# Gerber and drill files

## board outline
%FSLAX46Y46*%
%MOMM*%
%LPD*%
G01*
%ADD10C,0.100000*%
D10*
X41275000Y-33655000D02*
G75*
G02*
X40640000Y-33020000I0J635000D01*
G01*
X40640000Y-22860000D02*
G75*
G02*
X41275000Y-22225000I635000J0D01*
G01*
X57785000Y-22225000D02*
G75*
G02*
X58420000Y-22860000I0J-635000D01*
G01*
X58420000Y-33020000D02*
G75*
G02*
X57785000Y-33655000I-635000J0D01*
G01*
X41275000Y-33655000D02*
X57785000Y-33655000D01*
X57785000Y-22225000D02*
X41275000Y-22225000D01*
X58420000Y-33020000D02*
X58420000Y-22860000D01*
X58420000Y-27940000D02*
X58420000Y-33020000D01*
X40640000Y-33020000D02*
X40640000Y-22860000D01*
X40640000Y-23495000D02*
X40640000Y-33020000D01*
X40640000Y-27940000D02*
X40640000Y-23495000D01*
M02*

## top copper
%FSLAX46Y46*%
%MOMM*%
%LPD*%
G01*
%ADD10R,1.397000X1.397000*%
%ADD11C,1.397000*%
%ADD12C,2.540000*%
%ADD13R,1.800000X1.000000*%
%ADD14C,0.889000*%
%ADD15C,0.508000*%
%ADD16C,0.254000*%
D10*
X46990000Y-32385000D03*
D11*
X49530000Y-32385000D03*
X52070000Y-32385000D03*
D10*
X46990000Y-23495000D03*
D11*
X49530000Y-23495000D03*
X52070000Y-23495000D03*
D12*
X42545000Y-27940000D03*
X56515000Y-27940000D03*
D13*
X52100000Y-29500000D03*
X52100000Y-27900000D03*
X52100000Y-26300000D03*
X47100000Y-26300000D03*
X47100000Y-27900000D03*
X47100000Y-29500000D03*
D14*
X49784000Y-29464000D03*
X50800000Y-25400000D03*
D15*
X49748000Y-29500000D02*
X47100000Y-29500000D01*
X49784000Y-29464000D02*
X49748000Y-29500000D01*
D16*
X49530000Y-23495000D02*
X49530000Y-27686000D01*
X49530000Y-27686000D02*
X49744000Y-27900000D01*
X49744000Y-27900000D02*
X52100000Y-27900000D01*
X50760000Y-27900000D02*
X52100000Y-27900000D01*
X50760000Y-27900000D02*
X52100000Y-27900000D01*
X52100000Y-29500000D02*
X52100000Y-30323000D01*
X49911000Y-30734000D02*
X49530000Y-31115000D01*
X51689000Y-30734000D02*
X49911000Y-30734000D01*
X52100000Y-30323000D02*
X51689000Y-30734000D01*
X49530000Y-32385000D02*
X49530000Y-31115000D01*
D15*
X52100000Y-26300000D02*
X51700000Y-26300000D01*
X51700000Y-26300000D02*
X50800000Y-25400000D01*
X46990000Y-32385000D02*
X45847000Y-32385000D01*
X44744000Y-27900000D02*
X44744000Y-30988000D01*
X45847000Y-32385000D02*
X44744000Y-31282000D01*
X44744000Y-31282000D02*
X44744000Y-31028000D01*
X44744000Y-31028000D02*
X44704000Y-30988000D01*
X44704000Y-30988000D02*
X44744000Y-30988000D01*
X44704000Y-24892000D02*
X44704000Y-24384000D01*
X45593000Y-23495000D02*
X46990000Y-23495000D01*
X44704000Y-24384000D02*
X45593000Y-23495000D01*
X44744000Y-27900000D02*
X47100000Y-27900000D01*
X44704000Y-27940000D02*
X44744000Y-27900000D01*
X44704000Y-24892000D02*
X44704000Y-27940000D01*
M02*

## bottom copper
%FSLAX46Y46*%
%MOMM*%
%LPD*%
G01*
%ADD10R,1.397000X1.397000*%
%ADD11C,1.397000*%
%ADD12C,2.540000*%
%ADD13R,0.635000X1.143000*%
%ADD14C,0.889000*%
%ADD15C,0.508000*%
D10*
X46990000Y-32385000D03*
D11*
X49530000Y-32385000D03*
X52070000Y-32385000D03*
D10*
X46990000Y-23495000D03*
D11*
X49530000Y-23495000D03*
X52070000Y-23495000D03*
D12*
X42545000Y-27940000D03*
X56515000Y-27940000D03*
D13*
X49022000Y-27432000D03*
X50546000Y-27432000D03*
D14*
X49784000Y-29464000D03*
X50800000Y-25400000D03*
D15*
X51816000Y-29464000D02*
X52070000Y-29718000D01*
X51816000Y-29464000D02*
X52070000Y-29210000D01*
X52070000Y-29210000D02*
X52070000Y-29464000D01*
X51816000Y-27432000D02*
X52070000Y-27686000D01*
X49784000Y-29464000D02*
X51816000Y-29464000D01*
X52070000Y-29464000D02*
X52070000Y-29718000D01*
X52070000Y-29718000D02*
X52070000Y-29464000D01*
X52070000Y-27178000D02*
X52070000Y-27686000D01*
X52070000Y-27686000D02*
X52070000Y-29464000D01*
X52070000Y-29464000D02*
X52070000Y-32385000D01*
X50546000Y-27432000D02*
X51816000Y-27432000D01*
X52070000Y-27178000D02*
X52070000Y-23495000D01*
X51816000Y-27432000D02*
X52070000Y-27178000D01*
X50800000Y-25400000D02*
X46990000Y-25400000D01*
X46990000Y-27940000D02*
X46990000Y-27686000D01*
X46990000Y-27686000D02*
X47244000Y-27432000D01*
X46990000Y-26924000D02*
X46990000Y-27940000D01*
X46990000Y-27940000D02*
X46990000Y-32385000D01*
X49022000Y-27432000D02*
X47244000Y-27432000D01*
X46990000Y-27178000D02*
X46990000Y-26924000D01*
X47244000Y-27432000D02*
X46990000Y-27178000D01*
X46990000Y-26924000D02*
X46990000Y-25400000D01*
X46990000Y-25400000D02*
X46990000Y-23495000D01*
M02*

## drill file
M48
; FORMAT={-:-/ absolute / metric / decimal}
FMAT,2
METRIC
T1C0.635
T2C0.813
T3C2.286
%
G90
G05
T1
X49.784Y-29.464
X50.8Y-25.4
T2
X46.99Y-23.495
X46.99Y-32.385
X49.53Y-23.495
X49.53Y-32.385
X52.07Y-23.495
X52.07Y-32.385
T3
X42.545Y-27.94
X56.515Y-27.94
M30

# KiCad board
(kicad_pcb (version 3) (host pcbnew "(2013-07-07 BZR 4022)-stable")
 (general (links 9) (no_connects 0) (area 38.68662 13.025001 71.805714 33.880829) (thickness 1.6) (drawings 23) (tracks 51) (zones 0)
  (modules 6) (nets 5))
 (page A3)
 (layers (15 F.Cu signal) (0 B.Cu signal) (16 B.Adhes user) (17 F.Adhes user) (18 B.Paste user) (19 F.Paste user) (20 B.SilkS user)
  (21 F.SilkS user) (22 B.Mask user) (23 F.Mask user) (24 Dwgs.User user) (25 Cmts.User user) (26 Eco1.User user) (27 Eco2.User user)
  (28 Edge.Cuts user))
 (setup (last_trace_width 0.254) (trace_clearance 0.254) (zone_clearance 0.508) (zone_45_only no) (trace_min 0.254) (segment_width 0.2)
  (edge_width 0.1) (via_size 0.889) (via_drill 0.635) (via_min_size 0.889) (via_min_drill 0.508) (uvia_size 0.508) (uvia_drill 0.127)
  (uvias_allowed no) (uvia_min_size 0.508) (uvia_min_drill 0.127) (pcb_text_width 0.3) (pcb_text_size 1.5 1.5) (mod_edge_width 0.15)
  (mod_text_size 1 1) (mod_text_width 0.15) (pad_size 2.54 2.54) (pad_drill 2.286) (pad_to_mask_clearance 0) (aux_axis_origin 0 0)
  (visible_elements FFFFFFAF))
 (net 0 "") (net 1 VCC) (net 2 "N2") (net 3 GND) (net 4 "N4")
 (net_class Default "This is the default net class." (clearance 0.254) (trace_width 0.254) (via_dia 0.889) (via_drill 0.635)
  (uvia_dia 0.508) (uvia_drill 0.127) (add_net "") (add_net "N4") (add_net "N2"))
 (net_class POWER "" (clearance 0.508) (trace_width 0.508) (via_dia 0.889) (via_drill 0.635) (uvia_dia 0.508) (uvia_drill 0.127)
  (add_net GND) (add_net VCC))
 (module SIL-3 (layer F.Cu) (at 49.53 32.385)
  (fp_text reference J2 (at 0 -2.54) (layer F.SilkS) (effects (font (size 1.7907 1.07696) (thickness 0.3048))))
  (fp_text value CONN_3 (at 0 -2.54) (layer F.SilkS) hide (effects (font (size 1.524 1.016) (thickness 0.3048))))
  (pad 1 thru_hole rect (at -2.54 0) (size 1.397 1.397) (drill 0.8128) (layers *.Cu *.Mask F.SilkS) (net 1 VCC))
  (pad 2 thru_hole circle (at 0 0) (size 1.397 1.397) (drill 0.8128) (layers *.Cu *.Mask F.SilkS) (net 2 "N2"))
  (pad 3 thru_hole circle (at 2.54 0) (size 1.397 1.397) (drill 0.8128) (layers *.Cu *.Mask F.SilkS) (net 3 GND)))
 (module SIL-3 (layer F.Cu) (at 49.53 23.495)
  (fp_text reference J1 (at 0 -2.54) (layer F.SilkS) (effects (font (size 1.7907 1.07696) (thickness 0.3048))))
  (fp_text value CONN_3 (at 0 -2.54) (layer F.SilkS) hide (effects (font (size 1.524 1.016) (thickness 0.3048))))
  (pad 1 thru_hole rect (at -2.54 0) (size 1.397 1.397) (drill 0.8128) (layers *.Cu *.Mask F.SilkS) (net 1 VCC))
  (pad 2 thru_hole circle (at 0 0) (size 1.397 1.397) (drill 0.8128) (layers *.Cu *.Mask F.SilkS) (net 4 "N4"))
  (pad 3 thru_hole circle (at 2.54 0) (size 1.397 1.397) (drill 0.8128) (layers *.Cu *.Mask F.SilkS) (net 3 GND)))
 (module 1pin (layer F.Cu) (at 42.545 27.94)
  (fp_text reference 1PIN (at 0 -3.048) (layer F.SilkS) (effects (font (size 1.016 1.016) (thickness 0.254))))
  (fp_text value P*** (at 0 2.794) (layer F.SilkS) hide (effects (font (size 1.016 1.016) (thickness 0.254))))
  (pad 1 thru_hole circle (at 0 0) (size 2.54 2.54) (drill 2.286) (layers *.Cu *.Mask F.SilkS)))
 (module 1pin (layer F.Cu) (at 56.515 27.94)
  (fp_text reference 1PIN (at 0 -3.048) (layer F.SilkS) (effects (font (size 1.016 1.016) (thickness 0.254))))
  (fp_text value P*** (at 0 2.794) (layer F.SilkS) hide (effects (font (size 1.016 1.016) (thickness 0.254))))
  (pad 1 thru_hole circle (at 0 0) (size 2.54 2.54) (drill 2.286) (layers *.Cu *.Mask F.SilkS)))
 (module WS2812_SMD (layer F.Cu) (at 52.1 29.5)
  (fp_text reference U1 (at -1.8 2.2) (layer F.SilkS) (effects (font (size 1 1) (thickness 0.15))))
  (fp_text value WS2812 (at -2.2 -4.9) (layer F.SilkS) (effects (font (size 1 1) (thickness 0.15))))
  (pad 1 smd rect (at 0 0) (size 1.8 1) (layers F.Cu F.Paste F.Mask) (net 2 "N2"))
  (pad 2 smd rect (at 0 -1.6) (size 1.8 1) (layers F.Cu F.Paste F.Mask) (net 4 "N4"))
  (pad 3 smd rect (at 0 -3.2) (size 1.8 1) (layers F.Cu F.Paste F.Mask) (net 1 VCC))
  (pad 4 smd rect (at -5 -3.2) (size 1.8 1) (layers F.Cu F.Paste F.Mask))
  (pad 5 smd rect (at -5 -1.6) (size 1.8 1) (layers F.Cu F.Paste F.Mask) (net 1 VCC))
  (pad 6 smd rect (at -5 0) (size 1.8 1) (layers F.Cu F.Paste F.Mask) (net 3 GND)))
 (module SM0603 (layer B.Cu) (at 49.784 27.432)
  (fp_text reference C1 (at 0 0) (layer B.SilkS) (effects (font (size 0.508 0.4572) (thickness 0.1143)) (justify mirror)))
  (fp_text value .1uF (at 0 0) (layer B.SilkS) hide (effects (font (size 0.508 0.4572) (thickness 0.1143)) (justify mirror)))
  (pad 1 smd rect (at -0.762 0) (size 0.635 1.143) (layers B.Cu B.Paste B.Mask) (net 1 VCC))
  (pad 2 smd rect (at 0.762 0) (size 0.635 1.143) (layers B.Cu B.Paste B.Mask) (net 3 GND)))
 (gr_arc (start 41.275 33.02) (end 41.275 33.655) (angle 90) (layer Edge.Cuts) (width 0.1))
 (gr_arc (start 41.275 22.86) (end 40.64 22.86) (angle 90) (layer Edge.Cuts) (width 0.1))
 (gr_arc (start 57.785 22.86) (end 57.785 22.225) (angle 90) (layer Edge.Cuts) (width 0.1))
 (gr_arc (start 57.785 33.02) (end 58.42 33.02) (angle 90) (layer Edge.Cuts) (width 0.1))
 (gr_line (start 41.275 33.655) (end 57.785 33.655) (angle 90) (layer Edge.Cuts) (width 0.1))
 (gr_line (start 57.785 22.225) (end 41.275 22.225) (angle 90) (layer Edge.Cuts) (width 0.1))
 (gr_line (start 58.42 33.02) (end 58.42 22.86) (angle 90) (layer Edge.Cuts) (width 0.1))
 (gr_line (start 58.42 27.94) (end 58.42 33.02) (angle 90) (layer Edge.Cuts) (width 0.1))
 (gr_line (start 40.64 33.02) (end 40.64 22.86) (angle 90) (layer Edge.Cuts) (width 0.1))
 (gr_line (start 40.64 23.495) (end 40.64 33.02) (angle 90) (layer Edge.Cuts) (width 0.1))
 (gr_line (start 40.64 27.94) (end 40.64 23.495) (angle 90) (layer Edge.Cuts) (width 0.1))
 (segment (start 51.816 29.464) (end 52.07 29.718) (width 0.508) (layer B.Cu) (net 3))
 (segment (start 51.816 29.464) (end 52.07 29.21) (width 0.508) (layer B.Cu) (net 3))
 (segment (start 52.07 29.21) (end 52.07 29.464) (width 0.508) (layer B.Cu) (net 3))
 (segment (start 51.816 27.432) (end 52.07 27.686) (width 0.508) (layer B.Cu) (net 3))
 (segment (start 49.784 29.464) (end 51.816 29.464) (width 0.508) (layer B.Cu) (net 3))
 (segment (start 52.07 29.464) (end 52.07 29.718) (width 0.508) (layer B.Cu) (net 3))
 (segment (start 52.07 29.718) (end 52.07 29.464) (width 0.508) (layer B.Cu) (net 3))
 (segment (start 52.07 27.178) (end 52.07 27.686) (width 0.508) (layer B.Cu) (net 3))
 (segment (start 52.07 27.686) (end 52.07 29.464) (width 0.508) (layer B.Cu) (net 3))
 (segment (start 52.07 29.464) (end 52.07 32.385) (width 0.508) (layer B.Cu) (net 3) (status 800000))
 (segment (start 49.748 29.5) (end 47.1 29.5) (width 0.508) (layer F.Cu) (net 3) (status 800000))
 (segment (start 49.784 29.464) (end 49.748 29.5) (width 0.508) (layer F.Cu) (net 3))
 (via (at 49.784 29.464) (size 0.889) (layers F.Cu B.Cu) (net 3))
 (segment (start 50.546 27.432) (end 51.816 27.432) (width 0.508) (layer B.Cu) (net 3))
 (segment (start 52.07 27.178) (end 52.07 23.495) (width 0.508) (layer B.Cu) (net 3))
 (segment (start 51.816 27.432) (end 52.07 27.178) (width 0.508) (layer B.Cu) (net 3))
 (segment (start 49.53 23.495) (end 49.53 27.686) (width 0.254) (layer F.Cu) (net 4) (status 400000))
 (segment (start 49.53 27.686) (end 49.744 27.9) (width 0.254) (layer F.Cu) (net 4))
 (segment (start 49.744 27.9) (end 52.1 27.9) (width 0.254) (layer F.Cu) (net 4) (status 800000))
 (segment (start 50.76 27.9) (end 52.1 27.9) (width 0.254) (layer F.Cu) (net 4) (status 800000))
 (segment (start 50.76 27.9) (end 52.1 27.9) (width 0.254) (layer F.Cu) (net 4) (status 800000))
 (segment (start 52.1 29.5) (end 52.1 30.323) (width 0.254) (layer F.Cu) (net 2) (status 400000))
 (segment (start 49.911 30.734) (end 49.53 31.115) (width 0.254) (layer F.Cu) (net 2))
 (segment (start 51.689 30.734) (end 49.911 30.734) (width 0.254) (layer F.Cu) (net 2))
 (segment (start 52.1 30.323) (end 51.689 30.734) (width 0.254) (layer F.Cu) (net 2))
 (segment (start 49.53 32.385) (end 49.53 31.115) (width 0.254) (layer F.Cu) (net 2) (status 400000))
 (segment (start 52.1 26.3) (end 51.7 26.3) (width 0.508) (layer F.Cu) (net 1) (status C00000))
 (segment (start 50.8 25.4) (end 46.99 25.4) (width 0.508) (layer B.Cu) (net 1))
 (via (at 50.8 25.4) (size 0.889) (layers F.Cu B.Cu) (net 1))
 (segment (start 51.7 26.3) (end 50.8 25.4) (width 0.508) (layer F.Cu) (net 1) (status 400000))
 (segment (start 46.99 27.94) (end 46.99 27.686) (width 0.508) (layer B.Cu) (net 1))
 (segment (start 46.99 27.686) (end 47.244 27.432) (width 0.508) (layer B.Cu) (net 1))
 (segment (start 46.99 26.924) (end 46.99 27.94) (width 0.508) (layer B.Cu) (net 1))
 (segment (start 46.99 27.94) (end 46.99 32.385) (width 0.508) (layer B.Cu) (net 1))
 (segment (start 49.022 27.432) (end 47.244 27.432) (width 0.508) (layer B.Cu) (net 1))
 (segment (start 46.99 27.178) (end 46.99 26.924) (width 0.508) (layer B.Cu) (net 1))
 (segment (start 47.244 27.432) (end 46.99 27.178) (width 0.508) (layer B.Cu) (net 1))
 (segment (start 46.99 26.924) (end 46.99 25.4) (width 0.508) (layer B.Cu) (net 1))
 (segment (start 46.99 25.4) (end 46.99 23.495) (width 0.508) (layer B.Cu) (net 1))
 (segment (start 46.99 32.385) (end 45.847 32.385) (width 0.508) (layer F.Cu) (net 1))
 (segment (start 44.744 27.9) (end 44.744 30.988) (width 0.508) (layer F.Cu) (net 1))
 (segment (start 45.847 32.385) (end 44.744 31.282) (width 0.508) (layer F.Cu) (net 1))
 (segment (start 44.744 31.282) (end 44.744 31.028) (width 0.508) (layer F.Cu) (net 1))
 (segment (start 44.744 31.028) (end 44.704 30.988) (width 0.508) (layer F.Cu) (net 1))
 (segment (start 44.704 30.988) (end 44.744 30.988) (width 0.508) (layer F.Cu) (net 1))
 (segment (start 44.704 24.892) (end 44.704 24.384) (width 0.508) (layer F.Cu) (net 1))
 (segment (start 45.593 23.495) (end 46.99 23.495) (width 0.508) (layer F.Cu) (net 1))
 (segment (start 44.704 24.384) (end 45.593 23.495) (width 0.508) (layer F.Cu) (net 1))
 (segment (start 44.744 27.9) (end 47.1 27.9) (width 0.508) (layer F.Cu) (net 1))
 (segment (start 44.704 27.94) (end 44.744 27.9) (width 0.508) (layer F.Cu) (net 1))
 (segment (start 44.704 24.892) (end 44.704 27.94) (width 0.508) (layer F.Cu) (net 1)))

